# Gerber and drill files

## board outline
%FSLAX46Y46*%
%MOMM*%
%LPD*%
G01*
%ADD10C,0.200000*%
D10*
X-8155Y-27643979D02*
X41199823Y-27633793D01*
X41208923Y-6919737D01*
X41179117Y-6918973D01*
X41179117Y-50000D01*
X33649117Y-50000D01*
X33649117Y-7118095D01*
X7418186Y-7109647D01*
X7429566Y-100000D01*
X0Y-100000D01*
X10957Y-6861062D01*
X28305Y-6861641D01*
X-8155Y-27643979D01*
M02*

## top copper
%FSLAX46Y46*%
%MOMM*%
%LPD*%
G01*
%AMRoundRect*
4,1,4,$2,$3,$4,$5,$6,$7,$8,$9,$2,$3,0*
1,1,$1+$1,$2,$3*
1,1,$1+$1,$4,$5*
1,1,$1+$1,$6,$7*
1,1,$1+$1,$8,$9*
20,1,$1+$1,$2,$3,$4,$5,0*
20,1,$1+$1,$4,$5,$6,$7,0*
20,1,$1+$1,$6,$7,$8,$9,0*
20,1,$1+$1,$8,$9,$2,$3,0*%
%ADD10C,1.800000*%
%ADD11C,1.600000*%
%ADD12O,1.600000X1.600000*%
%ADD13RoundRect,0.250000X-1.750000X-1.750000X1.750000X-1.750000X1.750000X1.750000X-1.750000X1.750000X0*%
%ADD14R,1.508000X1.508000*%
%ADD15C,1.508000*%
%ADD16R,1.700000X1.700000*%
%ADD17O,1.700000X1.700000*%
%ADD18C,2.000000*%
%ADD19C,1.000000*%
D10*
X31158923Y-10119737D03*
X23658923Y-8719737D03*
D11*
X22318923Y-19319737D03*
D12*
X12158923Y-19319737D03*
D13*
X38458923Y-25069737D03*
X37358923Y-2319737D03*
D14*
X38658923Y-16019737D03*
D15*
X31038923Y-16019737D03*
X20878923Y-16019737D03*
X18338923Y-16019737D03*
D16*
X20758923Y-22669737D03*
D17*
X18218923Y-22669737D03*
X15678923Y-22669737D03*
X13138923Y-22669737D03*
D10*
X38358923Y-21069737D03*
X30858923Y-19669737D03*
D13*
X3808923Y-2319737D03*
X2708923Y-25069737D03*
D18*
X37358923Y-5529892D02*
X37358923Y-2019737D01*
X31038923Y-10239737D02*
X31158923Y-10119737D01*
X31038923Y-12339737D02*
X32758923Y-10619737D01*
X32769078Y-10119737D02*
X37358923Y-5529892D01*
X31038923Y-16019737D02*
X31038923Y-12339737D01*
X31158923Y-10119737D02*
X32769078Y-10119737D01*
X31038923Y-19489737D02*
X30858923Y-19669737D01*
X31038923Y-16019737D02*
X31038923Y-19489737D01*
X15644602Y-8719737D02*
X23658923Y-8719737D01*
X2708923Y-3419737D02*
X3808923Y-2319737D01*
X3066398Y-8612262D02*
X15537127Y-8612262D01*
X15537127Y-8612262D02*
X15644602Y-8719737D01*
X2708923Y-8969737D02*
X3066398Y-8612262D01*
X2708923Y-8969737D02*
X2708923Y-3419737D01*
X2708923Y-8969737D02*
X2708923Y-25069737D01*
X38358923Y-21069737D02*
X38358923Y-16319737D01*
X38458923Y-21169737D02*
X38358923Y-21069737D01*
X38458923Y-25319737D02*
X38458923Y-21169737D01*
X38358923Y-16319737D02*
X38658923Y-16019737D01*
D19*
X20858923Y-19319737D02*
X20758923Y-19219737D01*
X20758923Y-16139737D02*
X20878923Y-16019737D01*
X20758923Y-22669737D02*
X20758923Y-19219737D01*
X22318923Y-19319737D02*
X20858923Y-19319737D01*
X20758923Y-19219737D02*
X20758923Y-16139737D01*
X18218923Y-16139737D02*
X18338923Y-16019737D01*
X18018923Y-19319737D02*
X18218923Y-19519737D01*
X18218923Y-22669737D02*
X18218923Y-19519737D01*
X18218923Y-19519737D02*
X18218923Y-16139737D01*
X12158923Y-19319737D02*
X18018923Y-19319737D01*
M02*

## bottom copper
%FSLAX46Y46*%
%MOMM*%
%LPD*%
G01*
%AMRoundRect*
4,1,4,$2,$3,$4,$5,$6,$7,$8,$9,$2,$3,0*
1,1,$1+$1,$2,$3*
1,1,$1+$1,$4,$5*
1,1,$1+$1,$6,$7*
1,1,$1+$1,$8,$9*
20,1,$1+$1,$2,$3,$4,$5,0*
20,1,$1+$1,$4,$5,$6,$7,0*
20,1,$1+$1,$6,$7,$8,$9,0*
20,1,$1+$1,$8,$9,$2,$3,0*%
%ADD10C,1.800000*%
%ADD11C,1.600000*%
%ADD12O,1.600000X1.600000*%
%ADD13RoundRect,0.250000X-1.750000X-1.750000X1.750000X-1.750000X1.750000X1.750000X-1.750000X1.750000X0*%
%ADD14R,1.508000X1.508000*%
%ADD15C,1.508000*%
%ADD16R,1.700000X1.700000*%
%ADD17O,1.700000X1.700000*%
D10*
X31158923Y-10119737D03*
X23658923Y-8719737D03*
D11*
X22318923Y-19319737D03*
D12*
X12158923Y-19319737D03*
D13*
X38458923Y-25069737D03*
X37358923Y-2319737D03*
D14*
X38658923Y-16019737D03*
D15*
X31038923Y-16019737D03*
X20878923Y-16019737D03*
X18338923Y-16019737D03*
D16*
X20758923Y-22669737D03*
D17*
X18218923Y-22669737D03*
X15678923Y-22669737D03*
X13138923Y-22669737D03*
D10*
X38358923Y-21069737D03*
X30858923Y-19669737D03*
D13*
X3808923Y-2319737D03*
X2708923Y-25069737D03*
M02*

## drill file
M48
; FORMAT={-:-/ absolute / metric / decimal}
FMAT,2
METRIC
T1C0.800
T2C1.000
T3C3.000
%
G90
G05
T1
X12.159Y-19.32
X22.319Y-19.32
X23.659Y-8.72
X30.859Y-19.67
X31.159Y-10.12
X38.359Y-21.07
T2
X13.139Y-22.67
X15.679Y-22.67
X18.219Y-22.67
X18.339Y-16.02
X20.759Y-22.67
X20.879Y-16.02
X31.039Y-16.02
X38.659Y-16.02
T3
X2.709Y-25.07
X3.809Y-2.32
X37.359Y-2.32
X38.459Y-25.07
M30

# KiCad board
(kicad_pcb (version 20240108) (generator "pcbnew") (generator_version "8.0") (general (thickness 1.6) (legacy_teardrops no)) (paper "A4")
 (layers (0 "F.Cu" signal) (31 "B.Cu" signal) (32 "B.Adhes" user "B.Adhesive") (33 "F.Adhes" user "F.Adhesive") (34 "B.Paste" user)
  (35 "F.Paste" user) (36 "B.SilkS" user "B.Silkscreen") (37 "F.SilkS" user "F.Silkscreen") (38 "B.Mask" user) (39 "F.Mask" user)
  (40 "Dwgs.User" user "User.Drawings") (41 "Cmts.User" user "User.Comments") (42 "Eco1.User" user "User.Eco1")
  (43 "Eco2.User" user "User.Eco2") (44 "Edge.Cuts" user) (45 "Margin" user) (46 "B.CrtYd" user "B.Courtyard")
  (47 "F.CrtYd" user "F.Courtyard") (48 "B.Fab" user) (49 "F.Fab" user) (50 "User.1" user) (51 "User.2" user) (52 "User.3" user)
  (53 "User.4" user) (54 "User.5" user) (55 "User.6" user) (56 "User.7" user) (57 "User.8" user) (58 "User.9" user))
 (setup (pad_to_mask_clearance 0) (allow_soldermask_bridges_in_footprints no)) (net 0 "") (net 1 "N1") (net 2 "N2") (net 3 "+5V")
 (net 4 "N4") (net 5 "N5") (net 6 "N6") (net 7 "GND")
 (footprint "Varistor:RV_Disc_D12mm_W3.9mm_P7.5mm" (layer "F.Cu") (at 31.158923 10.119737 180)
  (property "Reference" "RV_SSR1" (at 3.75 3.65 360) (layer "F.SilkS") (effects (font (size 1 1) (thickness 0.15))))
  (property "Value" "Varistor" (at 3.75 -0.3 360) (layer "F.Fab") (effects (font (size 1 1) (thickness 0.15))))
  (pad "1" thru_hole circle (at 0 0 180) (size 1.8 1.8) (drill 0.8) (layers "*.Cu" "*.Mask") (remove_unused_layers no) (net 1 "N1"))
  (pad "2" thru_hole circle (at 7.5 1.4 180) (size 1.8 1.8) (drill 0.8) (layers "*.Cu" "*.Mask") (remove_unused_layers no) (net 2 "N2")))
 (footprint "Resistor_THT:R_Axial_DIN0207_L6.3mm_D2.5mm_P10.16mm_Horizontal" (layer "F.Cu") (at 22.318923 19.319737 180)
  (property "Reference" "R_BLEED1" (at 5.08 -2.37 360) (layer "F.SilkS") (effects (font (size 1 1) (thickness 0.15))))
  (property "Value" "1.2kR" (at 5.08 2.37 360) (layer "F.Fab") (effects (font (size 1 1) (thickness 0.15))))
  (pad "1" thru_hole circle (at 0 0 180) (size 1.6 1.6) (drill 0.8) (layers "*.Cu" "*.Mask") (remove_unused_layers no) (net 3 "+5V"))
  (pad "2" thru_hole oval (at 10.16 0 180) (size 1.6 1.6) (drill 0.8) (layers "*.Cu" "*.Mask") (remove_unused_layers no) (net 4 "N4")))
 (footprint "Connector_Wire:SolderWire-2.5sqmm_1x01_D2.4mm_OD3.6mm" (layer "F.Cu") (at 38.458923 25.069737)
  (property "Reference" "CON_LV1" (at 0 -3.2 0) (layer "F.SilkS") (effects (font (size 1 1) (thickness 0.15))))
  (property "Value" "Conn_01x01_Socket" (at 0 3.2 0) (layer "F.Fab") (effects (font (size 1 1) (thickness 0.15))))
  (pad "1" thru_hole roundrect (at 0 0) (size 4 4) (drill 3) (layers "*.Cu" "*.Mask") (remove_unused_layers no) (roundrect_rratio 0.0625)
   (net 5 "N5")))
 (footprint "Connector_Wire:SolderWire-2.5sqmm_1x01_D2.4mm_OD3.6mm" (layer "F.Cu") (at 37.358923 2.319737)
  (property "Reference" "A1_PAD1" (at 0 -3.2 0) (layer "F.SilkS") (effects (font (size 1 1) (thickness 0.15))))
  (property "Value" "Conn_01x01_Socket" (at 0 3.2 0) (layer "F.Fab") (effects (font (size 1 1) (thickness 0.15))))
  (pad "1" thru_hole roundrect (at 0 0) (size 4 4) (drill 3) (layers "*.Cu" "*.Mask") (remove_unused_layers no) (roundrect_rratio 0.0625)
   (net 1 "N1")))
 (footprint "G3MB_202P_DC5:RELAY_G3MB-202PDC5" (layer "F.Cu") (at 28.498923 14.619737 180)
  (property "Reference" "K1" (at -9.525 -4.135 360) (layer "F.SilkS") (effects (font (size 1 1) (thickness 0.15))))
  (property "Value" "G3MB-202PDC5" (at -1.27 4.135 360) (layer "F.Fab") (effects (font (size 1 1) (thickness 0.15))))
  (pad "1" thru_hole rect (at -10.16 -1.4 180) (size 1.508 1.508) (drill 1) (layers "*.Cu" "*.Mask") (remove_unused_layers no) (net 5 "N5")
   (solder_mask_margin 0.102))
  (pad "2" thru_hole circle (at -2.54 -1.4 180) (size 1.508 1.508) (drill 1) (layers "*.Cu" "*.Mask") (remove_unused_layers no) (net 1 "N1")
   (solder_mask_margin 0.102))
  (pad "3" thru_hole circle (at 7.62 -1.4 180) (size 1.508 1.508) (drill 1) (layers "*.Cu" "*.Mask") (remove_unused_layers no) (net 3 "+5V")
   (solder_mask_margin 0.102))
  (pad "4" thru_hole circle (at 10.16 -1.4 180) (size 1.508 1.508) (drill 1) (layers "*.Cu" "*.Mask") (remove_unused_layers no) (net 4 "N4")
   (solder_mask_margin 0.102)))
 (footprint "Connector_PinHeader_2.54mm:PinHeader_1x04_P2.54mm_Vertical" (layer "F.Cu") (at 20.758923 22.669737 -90)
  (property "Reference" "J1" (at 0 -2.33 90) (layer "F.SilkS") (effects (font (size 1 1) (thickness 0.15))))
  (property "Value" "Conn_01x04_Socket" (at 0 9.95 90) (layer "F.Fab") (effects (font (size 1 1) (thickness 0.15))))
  (pad "1" thru_hole rect (at 0 0 270) (size 1.7 1.7) (drill 1) (layers "*.Cu" "*.Mask") (remove_unused_layers no) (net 3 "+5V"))
  (pad "2" thru_hole oval (at 0 2.54 270) (size 1.7 1.7) (drill 1) (layers "*.Cu" "*.Mask") (remove_unused_layers no) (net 4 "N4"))
  (pad "3" thru_hole oval (at 0 5.08 270) (size 1.7 1.7) (drill 1) (layers "*.Cu" "*.Mask") (remove_unused_layers no) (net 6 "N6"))
  (pad "4" thru_hole oval (at 0 7.62 270) (size 1.7 1.7) (drill 1) (layers "*.Cu" "*.Mask") (remove_unused_layers no) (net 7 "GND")))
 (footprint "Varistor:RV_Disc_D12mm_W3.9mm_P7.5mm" (layer "F.Cu") (at 38.358923 21.069737 180)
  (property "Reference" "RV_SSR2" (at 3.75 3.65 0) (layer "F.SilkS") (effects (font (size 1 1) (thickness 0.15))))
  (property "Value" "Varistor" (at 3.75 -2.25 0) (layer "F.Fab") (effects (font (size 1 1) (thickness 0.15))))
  (pad "1" thru_hole circle (at 0 0 180) (size 1.8 1.8) (drill 0.8) (layers "*.Cu" "*.Mask") (remove_unused_layers no) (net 5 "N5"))
  (pad "2" thru_hole circle (at 7.5 1.4 180) (size 1.8 1.8) (drill 0.8) (layers "*.Cu" "*.Mask") (remove_unused_layers no) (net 1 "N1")))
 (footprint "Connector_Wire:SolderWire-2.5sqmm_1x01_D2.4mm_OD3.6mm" (layer "F.Cu") (at 3.808923 2.319737)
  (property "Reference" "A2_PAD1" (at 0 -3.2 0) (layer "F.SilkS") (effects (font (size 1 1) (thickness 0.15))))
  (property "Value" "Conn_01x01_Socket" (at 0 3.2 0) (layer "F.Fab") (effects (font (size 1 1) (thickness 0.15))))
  (pad "1" thru_hole roundrect (at 0 0) (size 4 4) (drill 3) (layers "*.Cu" "*.Mask") (remove_unused_layers no) (roundrect_rratio 0.0625)
   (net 2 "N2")))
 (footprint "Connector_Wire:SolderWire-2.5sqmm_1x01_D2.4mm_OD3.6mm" (layer "F.Cu") (at 2.708923 25.069737)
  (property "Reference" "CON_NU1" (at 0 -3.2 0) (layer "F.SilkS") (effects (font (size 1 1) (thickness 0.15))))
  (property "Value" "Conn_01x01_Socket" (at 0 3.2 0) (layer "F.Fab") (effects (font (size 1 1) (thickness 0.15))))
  (pad "1" thru_hole roundrect (at 0 0) (size 4 4) (drill 3) (layers "*.Cu" "*.Mask") (remove_unused_layers no) (roundrect_rratio 0.0625)
   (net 2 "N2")))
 (gr_poly
  (pts (xy -0.008155 27.643979) (xy 41.199823 27.633793) (xy 41.208923 6.919737) (xy 41.179117 6.918973) (xy 41.179117 0.05)
   (xy 33.649117 0.05) (xy 33.649117 7.118095) (xy 7.418186 7.109647) (xy 7.429566 0.1) (xy 0 0.1) (xy 0.010957 6.861062)
   (xy 0.028305 6.861641))
  (stroke (width 0.2) (type solid)) (fill none) (layer "Edge.Cuts"))
 (segment (start 37.358923 5.529892) (end 37.358923 2.019737) (width 2) (layer "F.Cu") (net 1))
 (segment (start 31.038923 10.239737) (end 31.158923 10.119737) (width 2) (layer "F.Cu") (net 1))
 (segment (start 31.038923 12.339737) (end 32.758923 10.619737) (width 2) (layer "F.Cu") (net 1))
 (segment (start 32.769078 10.119737) (end 37.358923 5.529892) (width 2) (layer "F.Cu") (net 1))
 (segment (start 31.038923 16.019737) (end 31.038923 12.339737) (width 2) (layer "F.Cu") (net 1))
 (segment (start 31.158923 10.119737) (end 32.769078 10.119737) (width 2) (layer "F.Cu") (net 1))
 (segment (start 31.038923 19.489737) (end 30.858923 19.669737) (width 2) (layer "F.Cu") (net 1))
 (segment (start 31.038923 16.019737) (end 31.038923 19.489737) (width 2) (layer "F.Cu") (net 1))
 (segment (start 15.644602 8.719737) (end 23.658923 8.719737) (width 2) (layer "F.Cu") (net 2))
 (segment (start 2.708923 3.419737) (end 3.808923 2.319737) (width 2) (layer "F.Cu") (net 2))
 (segment (start 3.066398 8.612262) (end 15.537127 8.612262) (width 2) (layer "F.Cu") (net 2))
 (segment (start 15.537127 8.612262) (end 15.644602 8.719737) (width 2) (layer "F.Cu") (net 2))
 (segment (start 2.708923 8.969737) (end 3.066398 8.612262) (width 2) (layer "F.Cu") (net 2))
 (segment (start 2.708923 8.969737) (end 2.708923 3.419737) (width 2) (layer "F.Cu") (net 2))
 (segment (start 2.708923 8.969737) (end 2.708923 25.069737) (width 2) (layer "F.Cu") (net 2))
 (segment (start 38.358923 21.069737) (end 38.358923 16.319737) (width 2) (layer "F.Cu") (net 5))
 (segment (start 38.458923 21.169737) (end 38.358923 21.069737) (width 2) (layer "F.Cu") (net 5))
 (segment (start 38.458923 25.319737) (end 38.458923 21.169737) (width 2) (layer "F.Cu") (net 5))
 (segment (start 38.358923 16.319737) (end 38.658923 16.019737) (width 2) (layer "F.Cu") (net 5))
 (segment (start 20.858923 19.319737) (end 20.758923 19.219737) (width 1) (layer "F.Cu") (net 3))
 (segment (start 20.758923 16.139737) (end 20.878923 16.019737) (width 1) (layer "F.Cu") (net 3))
 (segment (start 20.758923 22.669737) (end 20.758923 19.219737) (width 1) (layer "F.Cu") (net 3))
 (segment (start 22.318923 19.319737) (end 20.858923 19.319737) (width 1) (layer "F.Cu") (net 3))
 (segment (start 20.758923 19.219737) (end 20.758923 16.139737) (width 1) (layer "F.Cu") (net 3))
 (segment (start 18.218923 16.139737) (end 18.338923 16.019737) (width 1) (layer "F.Cu") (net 4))
 (segment (start 18.018923 19.319737) (end 18.218923 19.519737) (width 1) (layer "F.Cu") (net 4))
 (segment (start 18.218923 22.669737) (end 18.218923 19.519737) (width 1) (layer "F.Cu") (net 4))
 (segment (start 18.218923 19.519737) (end 18.218923 16.139737) (width 1) (layer "F.Cu") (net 4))
 (segment (start 12.158923 19.319737) (end 18.018923 19.319737) (width 1) (layer "F.Cu") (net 4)))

